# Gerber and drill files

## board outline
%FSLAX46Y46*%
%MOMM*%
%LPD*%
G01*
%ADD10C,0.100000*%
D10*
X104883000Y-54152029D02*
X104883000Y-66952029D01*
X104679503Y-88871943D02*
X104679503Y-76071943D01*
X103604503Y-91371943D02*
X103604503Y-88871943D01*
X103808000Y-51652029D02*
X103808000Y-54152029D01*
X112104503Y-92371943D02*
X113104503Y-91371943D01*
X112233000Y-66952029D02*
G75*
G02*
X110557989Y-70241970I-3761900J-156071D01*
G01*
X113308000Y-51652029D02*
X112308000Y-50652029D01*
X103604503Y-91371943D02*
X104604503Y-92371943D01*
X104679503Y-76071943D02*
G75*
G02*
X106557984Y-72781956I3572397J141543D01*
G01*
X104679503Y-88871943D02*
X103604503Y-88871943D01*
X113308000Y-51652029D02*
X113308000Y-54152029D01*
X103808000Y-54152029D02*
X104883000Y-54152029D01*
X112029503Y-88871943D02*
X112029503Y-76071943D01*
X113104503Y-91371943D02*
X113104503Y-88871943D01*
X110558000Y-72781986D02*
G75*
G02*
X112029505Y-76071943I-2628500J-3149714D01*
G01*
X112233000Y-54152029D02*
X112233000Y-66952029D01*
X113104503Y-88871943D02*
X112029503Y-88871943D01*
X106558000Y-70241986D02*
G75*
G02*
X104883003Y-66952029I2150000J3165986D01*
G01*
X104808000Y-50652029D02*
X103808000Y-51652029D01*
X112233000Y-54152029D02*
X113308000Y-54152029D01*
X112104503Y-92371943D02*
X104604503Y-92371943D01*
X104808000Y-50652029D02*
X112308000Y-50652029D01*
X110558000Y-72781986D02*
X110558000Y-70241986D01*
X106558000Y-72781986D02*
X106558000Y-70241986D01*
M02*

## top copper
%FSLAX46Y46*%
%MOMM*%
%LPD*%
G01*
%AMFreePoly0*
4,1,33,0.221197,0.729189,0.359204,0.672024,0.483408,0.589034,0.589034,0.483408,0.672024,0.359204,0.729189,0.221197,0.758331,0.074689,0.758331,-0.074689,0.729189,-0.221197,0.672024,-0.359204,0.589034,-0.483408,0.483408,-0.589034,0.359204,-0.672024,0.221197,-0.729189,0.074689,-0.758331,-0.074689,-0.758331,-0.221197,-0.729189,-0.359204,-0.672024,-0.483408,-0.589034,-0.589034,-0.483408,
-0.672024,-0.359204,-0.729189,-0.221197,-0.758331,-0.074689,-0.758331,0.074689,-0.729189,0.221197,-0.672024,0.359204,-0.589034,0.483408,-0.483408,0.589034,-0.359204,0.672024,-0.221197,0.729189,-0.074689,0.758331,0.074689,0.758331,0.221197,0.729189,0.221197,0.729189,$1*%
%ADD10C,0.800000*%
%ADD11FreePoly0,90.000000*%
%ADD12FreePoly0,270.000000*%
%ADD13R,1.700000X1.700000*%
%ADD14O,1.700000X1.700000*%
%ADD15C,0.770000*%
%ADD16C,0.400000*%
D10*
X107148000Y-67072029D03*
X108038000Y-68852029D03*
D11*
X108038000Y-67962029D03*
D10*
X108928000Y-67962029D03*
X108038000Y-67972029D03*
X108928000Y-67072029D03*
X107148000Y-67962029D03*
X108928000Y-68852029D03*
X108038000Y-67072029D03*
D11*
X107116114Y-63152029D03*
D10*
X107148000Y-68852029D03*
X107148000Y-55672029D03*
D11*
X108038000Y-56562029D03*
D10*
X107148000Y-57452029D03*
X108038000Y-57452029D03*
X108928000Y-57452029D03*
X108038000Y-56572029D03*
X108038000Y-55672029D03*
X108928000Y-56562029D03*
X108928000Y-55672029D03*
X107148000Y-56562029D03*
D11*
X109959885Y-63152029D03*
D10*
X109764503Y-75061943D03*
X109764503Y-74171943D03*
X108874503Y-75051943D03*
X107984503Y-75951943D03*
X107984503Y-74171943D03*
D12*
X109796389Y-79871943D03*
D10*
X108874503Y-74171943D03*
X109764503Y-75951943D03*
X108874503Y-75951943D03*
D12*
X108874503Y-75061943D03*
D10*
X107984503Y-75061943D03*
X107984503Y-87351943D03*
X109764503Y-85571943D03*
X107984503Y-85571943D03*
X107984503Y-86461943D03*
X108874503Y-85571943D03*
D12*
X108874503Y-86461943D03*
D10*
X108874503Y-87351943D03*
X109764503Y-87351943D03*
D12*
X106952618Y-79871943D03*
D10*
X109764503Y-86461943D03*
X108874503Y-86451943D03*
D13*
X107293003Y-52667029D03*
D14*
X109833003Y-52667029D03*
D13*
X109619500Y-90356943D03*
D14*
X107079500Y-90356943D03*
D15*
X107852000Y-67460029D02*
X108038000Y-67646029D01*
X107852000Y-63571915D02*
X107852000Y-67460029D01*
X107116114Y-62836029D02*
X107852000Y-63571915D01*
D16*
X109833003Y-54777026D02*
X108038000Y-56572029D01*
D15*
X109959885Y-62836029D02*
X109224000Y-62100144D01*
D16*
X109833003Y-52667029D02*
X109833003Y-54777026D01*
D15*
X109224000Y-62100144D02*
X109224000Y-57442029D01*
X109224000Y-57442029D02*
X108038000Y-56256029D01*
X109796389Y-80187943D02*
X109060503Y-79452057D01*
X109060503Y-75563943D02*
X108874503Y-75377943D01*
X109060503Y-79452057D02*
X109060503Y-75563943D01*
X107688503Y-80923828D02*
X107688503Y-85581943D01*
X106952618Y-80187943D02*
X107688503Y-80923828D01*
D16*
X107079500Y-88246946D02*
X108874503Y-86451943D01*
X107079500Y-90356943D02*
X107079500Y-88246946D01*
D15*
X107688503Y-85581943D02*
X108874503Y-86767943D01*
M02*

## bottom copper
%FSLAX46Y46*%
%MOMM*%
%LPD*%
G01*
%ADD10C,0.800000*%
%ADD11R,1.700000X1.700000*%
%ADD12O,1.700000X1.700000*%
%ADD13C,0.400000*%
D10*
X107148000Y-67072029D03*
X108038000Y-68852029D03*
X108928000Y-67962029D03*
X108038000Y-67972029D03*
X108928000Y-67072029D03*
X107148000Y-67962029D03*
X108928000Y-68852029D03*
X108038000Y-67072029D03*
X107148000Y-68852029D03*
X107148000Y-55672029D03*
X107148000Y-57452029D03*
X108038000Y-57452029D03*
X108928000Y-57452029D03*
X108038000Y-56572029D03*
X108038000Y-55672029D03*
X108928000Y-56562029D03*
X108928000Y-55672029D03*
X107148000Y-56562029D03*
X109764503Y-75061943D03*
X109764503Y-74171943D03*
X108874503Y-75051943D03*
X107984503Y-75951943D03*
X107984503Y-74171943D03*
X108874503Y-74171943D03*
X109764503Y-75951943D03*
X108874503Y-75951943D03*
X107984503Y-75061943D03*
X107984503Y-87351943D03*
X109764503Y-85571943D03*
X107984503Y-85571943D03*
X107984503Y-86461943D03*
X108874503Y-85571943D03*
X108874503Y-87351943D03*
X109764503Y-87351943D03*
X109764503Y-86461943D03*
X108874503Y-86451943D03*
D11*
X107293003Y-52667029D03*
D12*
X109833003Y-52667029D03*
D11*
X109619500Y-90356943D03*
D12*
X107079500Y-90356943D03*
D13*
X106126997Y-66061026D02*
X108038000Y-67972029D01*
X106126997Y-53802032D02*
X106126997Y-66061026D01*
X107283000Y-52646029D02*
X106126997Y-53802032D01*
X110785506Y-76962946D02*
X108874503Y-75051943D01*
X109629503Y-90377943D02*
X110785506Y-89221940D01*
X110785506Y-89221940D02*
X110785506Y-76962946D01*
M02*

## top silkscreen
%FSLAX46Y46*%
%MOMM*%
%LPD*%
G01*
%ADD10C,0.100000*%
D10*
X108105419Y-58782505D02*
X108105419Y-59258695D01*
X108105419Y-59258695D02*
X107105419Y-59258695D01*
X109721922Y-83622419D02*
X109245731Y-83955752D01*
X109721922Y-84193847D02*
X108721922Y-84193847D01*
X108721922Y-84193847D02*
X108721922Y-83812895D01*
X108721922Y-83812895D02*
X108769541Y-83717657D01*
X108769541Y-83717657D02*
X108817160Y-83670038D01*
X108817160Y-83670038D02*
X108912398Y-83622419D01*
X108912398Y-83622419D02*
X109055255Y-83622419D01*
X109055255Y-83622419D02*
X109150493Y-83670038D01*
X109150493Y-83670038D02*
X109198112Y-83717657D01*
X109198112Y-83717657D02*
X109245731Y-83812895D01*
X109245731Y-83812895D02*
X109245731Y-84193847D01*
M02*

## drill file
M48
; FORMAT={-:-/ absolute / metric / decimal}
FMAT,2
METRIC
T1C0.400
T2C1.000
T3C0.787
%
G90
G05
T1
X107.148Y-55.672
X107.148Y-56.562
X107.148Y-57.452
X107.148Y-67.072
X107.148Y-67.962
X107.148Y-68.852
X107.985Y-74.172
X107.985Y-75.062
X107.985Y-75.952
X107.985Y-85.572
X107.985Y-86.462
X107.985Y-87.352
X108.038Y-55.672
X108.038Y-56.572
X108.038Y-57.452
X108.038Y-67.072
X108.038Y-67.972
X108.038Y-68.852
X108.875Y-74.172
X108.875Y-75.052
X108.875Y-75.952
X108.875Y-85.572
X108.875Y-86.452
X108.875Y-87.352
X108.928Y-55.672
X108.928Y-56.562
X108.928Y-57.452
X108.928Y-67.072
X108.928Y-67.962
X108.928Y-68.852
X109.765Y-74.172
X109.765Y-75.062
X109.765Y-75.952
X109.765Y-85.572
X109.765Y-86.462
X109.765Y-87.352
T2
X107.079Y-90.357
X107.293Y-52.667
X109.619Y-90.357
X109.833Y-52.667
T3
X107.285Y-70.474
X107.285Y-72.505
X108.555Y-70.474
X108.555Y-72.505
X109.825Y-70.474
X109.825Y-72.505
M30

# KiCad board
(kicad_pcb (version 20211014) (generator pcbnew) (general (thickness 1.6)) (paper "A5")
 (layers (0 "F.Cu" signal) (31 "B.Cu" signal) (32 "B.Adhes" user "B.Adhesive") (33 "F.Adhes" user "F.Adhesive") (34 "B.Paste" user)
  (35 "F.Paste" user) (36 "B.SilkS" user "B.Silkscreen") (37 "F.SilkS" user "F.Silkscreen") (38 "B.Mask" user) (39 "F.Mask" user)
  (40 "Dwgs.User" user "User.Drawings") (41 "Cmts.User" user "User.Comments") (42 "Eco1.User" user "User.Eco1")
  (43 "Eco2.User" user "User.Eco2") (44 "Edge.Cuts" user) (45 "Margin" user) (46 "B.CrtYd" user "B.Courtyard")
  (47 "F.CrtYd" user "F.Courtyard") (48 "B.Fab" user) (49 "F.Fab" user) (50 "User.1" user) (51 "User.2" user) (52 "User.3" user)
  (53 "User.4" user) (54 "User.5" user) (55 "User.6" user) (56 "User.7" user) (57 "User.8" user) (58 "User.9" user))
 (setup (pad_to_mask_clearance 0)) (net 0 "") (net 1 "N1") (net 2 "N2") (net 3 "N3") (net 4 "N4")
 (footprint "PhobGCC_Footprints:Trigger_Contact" (layer "F.Cu") (at 108.538 63.152029 90)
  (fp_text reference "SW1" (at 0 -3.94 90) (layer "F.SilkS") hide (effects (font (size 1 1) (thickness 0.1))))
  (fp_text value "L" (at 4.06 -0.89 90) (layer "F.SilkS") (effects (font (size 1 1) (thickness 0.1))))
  (pad "1" thru_hole circle (at -3.92 -1.39 90) (size 0.8 0.8) (drill 0.4) (layers *.Cu *.Mask) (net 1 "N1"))
  (pad "1" thru_hole circle (at -5.7 -0.5 90) (size 0.8 0.8) (drill 0.4) (layers *.Cu *.Mask) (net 1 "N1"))
  (pad "1" smd custom (at -4.81 -0.5 90) (size 1.524 1.524) (layers "F.Cu" "F.Paste" "F.Mask") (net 1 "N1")
   (options (clearance outline) (anchor circle)) (primitives))
  (pad "1" thru_hole circle (at -4.81 0.39 90) (size 0.8 0.8) (drill 0.4) (layers *.Cu *.Mask) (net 1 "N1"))
  (pad "1" thru_hole circle (at -4.82 -0.5 90) (size 0.8 0.8) (drill 0.4) (layers *.Cu *.Mask) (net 1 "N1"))
  (pad "1" thru_hole circle (at -3.92 0.39 90) (size 0.8 0.8) (drill 0.4) (layers *.Cu *.Mask) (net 1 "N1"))
  (pad "1" thru_hole circle (at -4.81 -1.39 90) (size 0.8 0.8) (drill 0.4) (layers *.Cu *.Mask) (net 1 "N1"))
  (pad "1" thru_hole circle (at -5.7 0.39 90) (size 0.8 0.8) (drill 0.4) (layers *.Cu *.Mask) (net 1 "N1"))
  (pad "1" thru_hole circle (at -3.92 -0.5 90) (size 0.8 0.8) (drill 0.4) (layers *.Cu *.Mask) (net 1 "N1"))
  (pad "1" smd custom (at 0 -1.421886 90) (size 1.524 1.524) (layers "F.Cu" "F.Paste" "F.Mask") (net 1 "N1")
   (options (clearance outline) (anchor circle)) (primitives))
  (pad "1" thru_hole circle (at -5.7 -1.39 90) (size 0.8 0.8) (drill 0.4) (layers *.Cu *.Mask) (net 1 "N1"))
  (pad "2" thru_hole circle (at 7.48 -1.39 90) (size 0.8 0.8) (drill 0.4) (layers *.Cu *.Mask) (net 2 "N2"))
  (pad "2" smd custom (at 6.59 -0.5 90) (size 1.524 1.524) (layers "F.Cu" "F.Paste" "F.Mask") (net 2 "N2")
   (options (clearance outline) (anchor circle)) (primitives))
  (pad "2" thru_hole circle (at 5.7 -1.39 90) (size 0.8 0.8) (drill 0.4) (layers *.Cu *.Mask) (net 2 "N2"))
  (pad "2" thru_hole circle (at 5.7 -0.5 90) (size 0.8 0.8) (drill 0.4) (layers *.Cu *.Mask) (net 2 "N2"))
  (pad "2" thru_hole circle (at 5.7 0.39 90) (size 0.8 0.8) (drill 0.4) (layers *.Cu *.Mask) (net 2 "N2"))
  (pad "2" thru_hole circle (at 6.58 -0.5 90) (size 0.8 0.8) (drill 0.4) (layers *.Cu *.Mask) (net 2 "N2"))
  (pad "2" thru_hole circle (at 7.48 -0.5 90) (size 0.8 0.8) (drill 0.4) (layers *.Cu *.Mask) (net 2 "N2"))
  (pad "2" thru_hole circle (at 6.59 0.39 90) (size 0.8 0.8) (drill 0.4) (layers *.Cu *.Mask) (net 2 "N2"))
  (pad "2" thru_hole circle (at 7.48 0.39 90) (size 0.8 0.8) (drill 0.4) (layers *.Cu *.Mask) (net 2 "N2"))
  (pad "2" thru_hole circle (at 6.59 -1.39 90) (size 0.8 0.8) (drill 0.4) (layers *.Cu *.Mask) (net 2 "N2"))
  (pad "2" smd custom (at 0 1.421885 90) (size 1.524 1.524) (layers "F.Cu" "F.Paste" "F.Mask") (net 2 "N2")
   (options (clearance outline) (anchor circle)) (primitives)))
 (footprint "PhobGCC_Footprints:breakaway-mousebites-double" (layer "F.Cu") (at 108.325 70.244093 180)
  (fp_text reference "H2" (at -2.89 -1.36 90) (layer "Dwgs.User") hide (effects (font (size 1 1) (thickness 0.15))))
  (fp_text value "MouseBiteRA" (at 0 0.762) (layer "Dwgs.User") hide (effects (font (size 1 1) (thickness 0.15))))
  (fp_line (start -2.233 -2.537893) (end -2.233 0.002107) (layer "Edge.Cuts") (width 0.1))
  (fp_line (start 1.767 -2.537893) (end 1.767 0.002107) (layer "Edge.Cuts") (width 0.1))
  (pad "" np_thru_hole circle (at -0.23 -2.26085) (size 0.7874 0.7874) (drill 0.7874) (layers *.Cu *.Mask))
  (pad "" np_thru_hole circle (at 1.04 -0.23 180) (size 0.7874 0.7874) (drill 0.7874) (layers *.Cu *.Mask))
  (pad "" np_thru_hole circle (at -1.5 -0.23 180) (size 0.7874 0.7874) (drill 0.7874) (layers *.Cu *.Mask))
  (pad "" np_thru_hole circle (at -0.23 -0.23 180) (size 0.7874 0.7874) (drill 0.7874) (layers *.Cu *.Mask))
  (pad "" np_thru_hole circle (at 1.04 -2.26085) (size 0.7874 0.7874) (drill 0.7874) (layers *.Cu *.Mask))
  (pad "" np_thru_hole circle (at -1.5 -2.26085) (size 0.7874 0.7874) (drill 0.7874) (layers *.Cu *.Mask)))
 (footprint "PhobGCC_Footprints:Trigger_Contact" (layer "F.Cu") (at 108.374503 79.871943 -90)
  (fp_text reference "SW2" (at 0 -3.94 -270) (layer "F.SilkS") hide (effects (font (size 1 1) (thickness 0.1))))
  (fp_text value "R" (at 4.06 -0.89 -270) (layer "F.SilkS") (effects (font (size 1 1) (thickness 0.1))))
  (pad "1" thru_hole circle (at -4.81 -1.39 270) (size 0.8 0.8) (drill 0.4) (layers *.Cu *.Mask) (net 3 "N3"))
  (pad "1" thru_hole circle (at -5.7 -1.39 270) (size 0.8 0.8) (drill 0.4) (layers *.Cu *.Mask) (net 3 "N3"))
  (pad "1" thru_hole circle (at -4.82 -0.5 270) (size 0.8 0.8) (drill 0.4) (layers *.Cu *.Mask) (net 3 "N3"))
  (pad "1" thru_hole circle (at -3.92 0.39 270) (size 0.8 0.8) (drill 0.4) (layers *.Cu *.Mask) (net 3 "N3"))
  (pad "1" thru_hole circle (at -5.7 0.39 270) (size 0.8 0.8) (drill 0.4) (layers *.Cu *.Mask) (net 3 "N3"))
  (pad "1" smd custom (at 0 -1.421886 270) (size 1.524 1.524) (layers "F.Cu" "F.Paste" "F.Mask") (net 3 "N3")
   (options (clearance outline) (anchor circle)) (primitives))
  (pad "1" thru_hole circle (at -5.7 -0.5 270) (size 0.8 0.8) (drill 0.4) (layers *.Cu *.Mask) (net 3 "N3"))
  (pad "1" thru_hole circle (at -3.92 -1.39 270) (size 0.8 0.8) (drill 0.4) (layers *.Cu *.Mask) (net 3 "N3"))
  (pad "1" thru_hole circle (at -3.92 -0.5 270) (size 0.8 0.8) (drill 0.4) (layers *.Cu *.Mask) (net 3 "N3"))
  (pad "1" smd custom (at -4.81 -0.5 270) (size 1.524 1.524) (layers "F.Cu" "F.Paste" "F.Mask") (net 3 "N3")
   (options (clearance outline) (anchor circle)) (primitives))
  (pad "1" thru_hole circle (at -4.81 0.39 270) (size 0.8 0.8) (drill 0.4) (layers *.Cu *.Mask) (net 3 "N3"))
  (pad "2" thru_hole circle (at 7.48 0.39 270) (size 0.8 0.8) (drill 0.4) (layers *.Cu *.Mask) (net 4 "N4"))
  (pad "2" thru_hole circle (at 5.7 -1.39 270) (size 0.8 0.8) (drill 0.4) (layers *.Cu *.Mask) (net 4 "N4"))
  (pad "2" thru_hole circle (at 5.7 0.39 270) (size 0.8 0.8) (drill 0.4) (layers *.Cu *.Mask) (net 4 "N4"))
  (pad "2" thru_hole circle (at 6.59 0.39 270) (size 0.8 0.8) (drill 0.4) (layers *.Cu *.Mask) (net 4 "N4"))
  (pad "2" thru_hole circle (at 5.7 -0.5 270) (size 0.8 0.8) (drill 0.4) (layers *.Cu *.Mask) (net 4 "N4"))
  (pad "2" smd custom (at 6.59 -0.5 270) (size 1.524 1.524) (layers "F.Cu" "F.Paste" "F.Mask") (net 4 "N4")
   (options (clearance outline) (anchor circle)) (primitives))
  (pad "2" thru_hole circle (at 7.48 -0.5 270) (size 0.8 0.8) (drill 0.4) (layers *.Cu *.Mask) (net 4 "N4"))
  (pad "2" thru_hole circle (at 7.48 -1.39 270) (size 0.8 0.8) (drill 0.4) (layers *.Cu *.Mask) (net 4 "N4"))
  (pad "2" smd custom (at 0 1.421885 270) (size 1.524 1.524) (layers "F.Cu" "F.Paste" "F.Mask") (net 4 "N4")
   (options (clearance outline) (anchor circle)) (primitives))
  (pad "2" thru_hole circle (at 6.59 -1.39 270) (size 0.8 0.8) (drill 0.4) (layers *.Cu *.Mask) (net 4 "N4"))
  (pad "2" thru_hole circle (at 6.58 -0.5 270) (size 0.8 0.8) (drill 0.4) (layers *.Cu *.Mask) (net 4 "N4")))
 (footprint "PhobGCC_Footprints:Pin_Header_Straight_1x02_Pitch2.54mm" (layer "B.Cu") (at 107.293003 52.667029 -90)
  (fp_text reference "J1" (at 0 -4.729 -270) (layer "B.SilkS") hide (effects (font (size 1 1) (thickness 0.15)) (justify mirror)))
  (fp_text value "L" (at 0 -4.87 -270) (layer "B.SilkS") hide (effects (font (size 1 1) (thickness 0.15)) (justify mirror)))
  (pad "1" thru_hole rect (at 0 0 270) (size 1.7 1.7) (drill 1) (layers *.Cu *.Mask) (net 1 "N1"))
  (pad "2" thru_hole oval (at 0 -2.54 270) (size 1.7 1.7) (drill 1) (layers *.Cu *.Mask) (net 2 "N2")))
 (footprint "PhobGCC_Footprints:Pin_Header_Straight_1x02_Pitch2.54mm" (layer "B.Cu") (at 109.6195 90.356943 90)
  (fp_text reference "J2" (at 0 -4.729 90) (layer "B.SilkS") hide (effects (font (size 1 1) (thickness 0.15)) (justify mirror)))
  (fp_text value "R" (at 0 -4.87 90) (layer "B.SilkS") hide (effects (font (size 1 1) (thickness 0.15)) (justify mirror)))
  (pad "1" thru_hole rect (at 0 0 90) (size 1.7 1.7) (drill 1) (layers *.Cu *.Mask) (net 3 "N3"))
  (pad "2" thru_hole oval (at 0 -2.54 90) (size 1.7 1.7) (drill 1) (layers *.Cu *.Mask) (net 4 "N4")))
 (gr_line (start 104.883 54.152029) (end 104.883 66.952029) (layer "Edge.Cuts") (width 0.1))
 (gr_line (start 104.679503 88.871943) (end 104.679503 76.071943) (layer "Edge.Cuts") (width 0.1))
 (gr_line (start 103.604503 91.371943) (end 103.604503 88.871943) (layer "Edge.Cuts") (width 0.1))
 (gr_line (start 103.808 51.652029) (end 103.808 54.152029) (layer "Edge.Cuts") (width 0.1))
 (gr_line (start 112.104503 92.371943) (end 113.104503 91.371943) (layer "Edge.Cuts") (width 0.1))
 (gr_arc (start 112.233 66.952029) (mid 111.826403 68.816395) (end 110.558 70.241986) (layer "Edge.Cuts") (width 0.1))
 (gr_line (start 113.308 51.652029) (end 112.308 50.652029) (layer "Edge.Cuts") (width 0.1))
 (gr_line (start 103.604503 91.371943) (end 104.604503 92.371943) (layer "Edge.Cuts") (width 0.1))
 (gr_arc (start 104.679503 76.071943) (mid 105.14715 74.157693) (end 106.558 72.781986) (layer "Edge.Cuts") (width 0.1))
 (gr_line (start 104.679503 88.871943) (end 103.604503 88.871943) (layer "Edge.Cuts") (width 0.1))
 (gr_line (start 113.308 51.652029) (end 113.308 54.152029) (layer "Edge.Cuts") (width 0.1))
 (gr_line (start 103.808 54.152029) (end 104.883 54.152029) (layer "Edge.Cuts") (width 0.1))
 (gr_line (start 112.029503 88.871943) (end 112.029503 76.071943) (layer "Edge.Cuts") (width 0.1))
 (gr_line (start 113.104503 91.371943) (end 113.104503 88.871943) (layer "Edge.Cuts") (width 0.1))
 (gr_arc (start 110.558 72.781986) (mid 111.674383 74.256719) (end 112.029503 76.071943) (layer "Edge.Cuts") (width 0.1))
 (gr_line (start 112.233 54.152029) (end 112.233 66.952029) (layer "Edge.Cuts") (width 0.1))
 (gr_line (start 113.104503 88.871943) (end 112.029503 88.871943) (layer "Edge.Cuts") (width 0.1))
 (gr_arc (start 106.558 70.241986) (mid 105.297554 68.812335) (end 104.883 66.952029) (layer "Edge.Cuts") (width 0.1))
 (gr_line (start 104.808 50.652029) (end 103.808 51.652029) (layer "Edge.Cuts") (width 0.1))
 (gr_line (start 112.233 54.152029) (end 113.308 54.152029) (layer "Edge.Cuts") (width 0.1))
 (gr_line (start 112.104503 92.371943) (end 104.604503 92.371943) (layer "Edge.Cuts") (width 0.1))
 (gr_line (start 104.808 50.652029) (end 112.308 50.652029) (layer "Edge.Cuts") (width 0.1))
 (segment (start 107.852 67.460029) (end 108.038 67.646029) (width 0.77) (layer "F.Cu") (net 1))
 (segment (start 107.852 63.571915) (end 107.852 67.460029) (width 0.77) (layer "F.Cu") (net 1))
 (segment (start 107.116114 62.836029) (end 107.852 63.571915) (width 0.77) (layer "F.Cu") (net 1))
 (segment (start 106.126997 66.061026) (end 108.038 67.972029) (width 0.4) (layer "B.Cu") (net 1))
 (segment (start 106.126997 53.802032) (end 106.126997 66.061026) (width 0.4) (layer "B.Cu") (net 1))
 (segment (start 107.283 52.646029) (end 106.126997 53.802032) (width 0.4) (layer "B.Cu") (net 1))
 (segment (start 109.833003 54.777026) (end 108.038 56.572029) (width 0.4) (layer "F.Cu") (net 2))
 (segment (start 109.959885 62.836029) (end 109.224 62.100144) (width 0.77) (layer "F.Cu") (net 2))
 (segment (start 109.833003 52.667029) (end 109.833003 54.777026) (width 0.4) (layer "F.Cu") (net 2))
 (segment (start 109.224 62.100144) (end 109.224 57.442029) (width 0.77) (layer "F.Cu") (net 2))
 (segment (start 109.224 57.442029) (end 108.038 56.256029) (width 0.77) (layer "F.Cu") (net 2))
 (segment (start 109.796389 80.187943) (end 109.060503 79.452057) (width 0.77) (layer "F.Cu") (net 3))
 (segment (start 109.060503 75.563943) (end 108.874503 75.377943) (width 0.77) (layer "F.Cu") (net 3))
 (segment (start 109.060503 79.452057) (end 109.060503 75.563943) (width 0.77) (layer "F.Cu") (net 3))
 (segment (start 110.785506 76.962946) (end 108.874503 75.051943) (width 0.4) (layer "B.Cu") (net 3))
 (segment (start 109.629503 90.377943) (end 110.785506 89.22194) (width 0.4) (layer "B.Cu") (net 3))
 (segment (start 110.785506 89.22194) (end 110.785506 76.962946) (width 0.4) (layer "B.Cu") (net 3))
 (segment (start 107.688503 80.923828) (end 107.688503 85.581943) (width 0.77) (layer "F.Cu") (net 4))
 (segment (start 106.952618 80.187943) (end 107.688503 80.923828) (width 0.77) (layer "F.Cu") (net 4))
 (segment (start 107.0795 88.246946) (end 108.874503 86.451943) (width 0.4) (layer "F.Cu") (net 4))
 (segment (start 107.0795 90.356943) (end 107.0795 88.246946) (width 0.4) (layer "F.Cu") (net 4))
 (segment (start 107.688503 85.581943) (end 108.874503 86.767943) (width 0.77) (layer "F.Cu") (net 4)))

